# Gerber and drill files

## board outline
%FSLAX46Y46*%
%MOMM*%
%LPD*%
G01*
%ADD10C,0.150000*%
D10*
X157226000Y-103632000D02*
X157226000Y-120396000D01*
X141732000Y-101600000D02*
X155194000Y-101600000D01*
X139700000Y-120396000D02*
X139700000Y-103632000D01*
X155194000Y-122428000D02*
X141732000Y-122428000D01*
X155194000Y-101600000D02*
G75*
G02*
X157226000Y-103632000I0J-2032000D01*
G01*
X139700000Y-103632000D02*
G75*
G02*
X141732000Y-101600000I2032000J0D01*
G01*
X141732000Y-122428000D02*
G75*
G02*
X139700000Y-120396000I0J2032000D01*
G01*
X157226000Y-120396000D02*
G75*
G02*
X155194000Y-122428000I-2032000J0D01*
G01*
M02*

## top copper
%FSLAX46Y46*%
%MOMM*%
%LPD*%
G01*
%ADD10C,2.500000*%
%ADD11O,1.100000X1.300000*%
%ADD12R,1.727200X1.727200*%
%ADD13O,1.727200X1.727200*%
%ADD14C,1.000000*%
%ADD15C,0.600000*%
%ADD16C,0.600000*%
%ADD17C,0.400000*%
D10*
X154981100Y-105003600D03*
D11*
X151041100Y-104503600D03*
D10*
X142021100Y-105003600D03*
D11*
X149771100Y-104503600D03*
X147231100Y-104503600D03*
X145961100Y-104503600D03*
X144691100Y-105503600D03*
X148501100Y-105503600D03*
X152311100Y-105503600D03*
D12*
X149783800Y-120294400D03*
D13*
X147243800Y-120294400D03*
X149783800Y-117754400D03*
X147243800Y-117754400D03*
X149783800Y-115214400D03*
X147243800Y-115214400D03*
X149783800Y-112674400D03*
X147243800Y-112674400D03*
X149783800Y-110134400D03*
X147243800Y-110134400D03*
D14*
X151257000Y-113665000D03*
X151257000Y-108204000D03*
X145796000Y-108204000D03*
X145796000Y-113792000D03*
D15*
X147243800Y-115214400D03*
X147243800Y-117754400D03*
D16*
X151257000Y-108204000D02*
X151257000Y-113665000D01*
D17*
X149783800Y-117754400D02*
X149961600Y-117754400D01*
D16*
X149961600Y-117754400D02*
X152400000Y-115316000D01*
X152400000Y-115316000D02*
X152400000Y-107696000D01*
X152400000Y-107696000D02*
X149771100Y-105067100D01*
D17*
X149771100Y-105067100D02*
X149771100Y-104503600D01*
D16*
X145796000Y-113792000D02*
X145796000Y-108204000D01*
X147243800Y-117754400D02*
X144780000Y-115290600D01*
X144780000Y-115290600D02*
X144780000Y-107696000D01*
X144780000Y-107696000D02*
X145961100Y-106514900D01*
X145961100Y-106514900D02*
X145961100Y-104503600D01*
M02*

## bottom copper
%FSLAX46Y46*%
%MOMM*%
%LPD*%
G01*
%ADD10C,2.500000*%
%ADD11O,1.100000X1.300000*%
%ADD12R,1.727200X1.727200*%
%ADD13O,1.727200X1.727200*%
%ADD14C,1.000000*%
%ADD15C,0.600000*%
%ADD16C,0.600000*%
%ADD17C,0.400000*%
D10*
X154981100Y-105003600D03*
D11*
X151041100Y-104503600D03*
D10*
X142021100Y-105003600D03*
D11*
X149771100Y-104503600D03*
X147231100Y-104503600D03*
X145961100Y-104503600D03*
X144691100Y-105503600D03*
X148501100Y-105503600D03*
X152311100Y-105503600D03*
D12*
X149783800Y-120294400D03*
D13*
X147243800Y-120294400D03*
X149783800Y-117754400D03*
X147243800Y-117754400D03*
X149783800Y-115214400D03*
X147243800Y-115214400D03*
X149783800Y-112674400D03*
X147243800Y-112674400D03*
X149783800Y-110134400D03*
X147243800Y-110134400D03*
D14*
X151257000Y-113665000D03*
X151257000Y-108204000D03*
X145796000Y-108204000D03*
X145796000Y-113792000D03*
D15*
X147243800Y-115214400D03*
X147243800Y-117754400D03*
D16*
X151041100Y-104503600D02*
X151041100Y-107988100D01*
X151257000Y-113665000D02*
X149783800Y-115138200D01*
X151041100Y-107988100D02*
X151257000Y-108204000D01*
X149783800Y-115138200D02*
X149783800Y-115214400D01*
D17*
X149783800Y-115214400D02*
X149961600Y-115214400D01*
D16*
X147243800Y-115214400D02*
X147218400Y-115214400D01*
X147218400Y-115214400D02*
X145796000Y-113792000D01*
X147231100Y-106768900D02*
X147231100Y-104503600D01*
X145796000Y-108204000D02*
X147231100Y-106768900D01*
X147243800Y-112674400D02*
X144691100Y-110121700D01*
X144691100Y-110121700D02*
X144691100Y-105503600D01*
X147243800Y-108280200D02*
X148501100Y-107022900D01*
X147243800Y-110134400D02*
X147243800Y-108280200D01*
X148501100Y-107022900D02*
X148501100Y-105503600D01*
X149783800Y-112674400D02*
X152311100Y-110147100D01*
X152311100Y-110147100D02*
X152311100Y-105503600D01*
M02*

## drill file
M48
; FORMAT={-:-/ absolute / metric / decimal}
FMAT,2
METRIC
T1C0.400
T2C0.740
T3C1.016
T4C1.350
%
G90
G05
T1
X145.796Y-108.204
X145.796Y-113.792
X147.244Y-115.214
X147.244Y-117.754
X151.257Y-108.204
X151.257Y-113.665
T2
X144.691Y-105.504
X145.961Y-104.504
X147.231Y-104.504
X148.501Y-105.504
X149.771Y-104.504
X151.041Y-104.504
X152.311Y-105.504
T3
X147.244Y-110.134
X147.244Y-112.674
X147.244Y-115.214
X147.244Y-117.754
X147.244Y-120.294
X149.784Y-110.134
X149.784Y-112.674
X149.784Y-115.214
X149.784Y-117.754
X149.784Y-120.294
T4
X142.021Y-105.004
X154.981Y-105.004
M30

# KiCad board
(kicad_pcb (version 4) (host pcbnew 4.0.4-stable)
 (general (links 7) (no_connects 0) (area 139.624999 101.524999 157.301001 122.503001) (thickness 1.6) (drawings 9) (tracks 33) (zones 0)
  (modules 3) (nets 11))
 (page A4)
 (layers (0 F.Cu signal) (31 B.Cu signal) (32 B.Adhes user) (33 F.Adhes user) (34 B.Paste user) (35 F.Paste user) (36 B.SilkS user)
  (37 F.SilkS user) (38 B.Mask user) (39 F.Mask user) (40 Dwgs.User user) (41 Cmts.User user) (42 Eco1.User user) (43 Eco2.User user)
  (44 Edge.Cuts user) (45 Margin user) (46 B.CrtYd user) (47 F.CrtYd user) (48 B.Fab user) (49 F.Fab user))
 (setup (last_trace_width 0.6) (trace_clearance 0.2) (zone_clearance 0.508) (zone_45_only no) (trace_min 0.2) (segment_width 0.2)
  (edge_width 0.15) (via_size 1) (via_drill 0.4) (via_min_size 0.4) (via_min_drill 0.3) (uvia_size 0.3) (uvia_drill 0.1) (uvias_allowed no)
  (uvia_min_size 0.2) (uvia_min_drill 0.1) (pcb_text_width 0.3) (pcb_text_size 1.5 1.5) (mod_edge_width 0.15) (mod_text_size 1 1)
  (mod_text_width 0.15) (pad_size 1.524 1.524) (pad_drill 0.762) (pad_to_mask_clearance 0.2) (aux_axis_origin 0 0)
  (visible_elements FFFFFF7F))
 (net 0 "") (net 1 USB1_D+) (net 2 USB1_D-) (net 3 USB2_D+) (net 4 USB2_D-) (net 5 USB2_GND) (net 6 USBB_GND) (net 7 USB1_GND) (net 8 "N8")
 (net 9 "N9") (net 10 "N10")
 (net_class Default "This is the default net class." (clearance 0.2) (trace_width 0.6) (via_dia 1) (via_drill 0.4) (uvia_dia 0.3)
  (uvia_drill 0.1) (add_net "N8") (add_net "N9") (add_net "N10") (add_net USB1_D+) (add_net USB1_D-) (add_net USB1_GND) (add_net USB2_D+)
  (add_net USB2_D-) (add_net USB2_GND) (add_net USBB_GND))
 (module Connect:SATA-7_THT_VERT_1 (layer F.Cu) (at 148.5011 105.0036)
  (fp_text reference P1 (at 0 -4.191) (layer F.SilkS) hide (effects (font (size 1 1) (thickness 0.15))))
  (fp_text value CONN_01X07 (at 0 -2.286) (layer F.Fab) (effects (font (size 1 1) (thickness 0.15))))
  (pad 9 thru_hole circle (at 6.48 0) (size 2.5 2.5) (drill 1.35) (layers *.Cu *.Mask F.SilkS))
  (pad 2 thru_hole oval (at 2.54 -0.5) (size 1.1 1.3) (drill 0.74) (layers *.Cu *.Mask F.SilkS) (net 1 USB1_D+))
  (pad 8 thru_hole circle (at -6.48 0) (size 2.5 2.5) (drill 1.35) (layers *.Cu *.Mask F.SilkS))
  (pad 3 thru_hole oval (at 1.27 -0.5) (size 1.1 1.3) (drill 0.74) (layers *.Cu *.Mask F.SilkS) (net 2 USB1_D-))
  (pad 5 thru_hole oval (at -1.27 -0.5) (size 1.1 1.3) (drill 0.74) (layers *.Cu *.Mask F.SilkS) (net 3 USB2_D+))
  (pad 6 thru_hole oval (at -2.54 -0.5) (size 1.1 1.3) (drill 0.74) (layers *.Cu *.Mask F.SilkS) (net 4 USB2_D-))
  (pad 7 thru_hole oval (at -3.81 0.5) (size 1.1 1.3) (drill 0.74) (layers *.Cu *.Mask F.SilkS) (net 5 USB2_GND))
  (pad 4 thru_hole oval (at 0 0.5) (size 1.1 1.3) (drill 0.74) (layers *.Cu *.Mask F.SilkS) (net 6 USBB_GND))
  (pad 1 thru_hole oval (at 3.81 0.5) (size 1.1 1.3) (drill 0.74) (layers *.Cu *.Mask F.SilkS) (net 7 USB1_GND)))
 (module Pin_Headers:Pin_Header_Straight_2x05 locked (layer F.Cu) (at 149.7838 120.2944 180)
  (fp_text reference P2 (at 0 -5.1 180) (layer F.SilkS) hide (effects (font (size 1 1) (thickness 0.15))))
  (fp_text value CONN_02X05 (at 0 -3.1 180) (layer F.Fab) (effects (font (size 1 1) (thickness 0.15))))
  (pad 1 thru_hole rect (at 0 0 180) (size 1.7272 1.7272) (drill 1.016) (layers *.Cu *.Mask F.SilkS) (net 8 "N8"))
  (pad 2 thru_hole oval (at 2.54 0 180) (size 1.7272 1.7272) (drill 1.016) (layers *.Cu *.Mask F.SilkS) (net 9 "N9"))
  (pad 3 thru_hole oval (at 0 2.54 180) (size 1.7272 1.7272) (drill 1.016) (layers *.Cu *.Mask F.SilkS) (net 2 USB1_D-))
  (pad 4 thru_hole oval (at 2.54 2.54 180) (size 1.7272 1.7272) (drill 1.016) (layers *.Cu *.Mask F.SilkS) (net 4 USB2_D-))
  (pad 5 thru_hole oval (at 0 5.08 180) (size 1.7272 1.7272) (drill 1.016) (layers *.Cu *.Mask F.SilkS) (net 1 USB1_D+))
  (pad 6 thru_hole oval (at 2.54 5.08 180) (size 1.7272 1.7272) (drill 1.016) (layers *.Cu *.Mask F.SilkS) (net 3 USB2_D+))
  (pad 7 thru_hole oval (at 0 7.62 180) (size 1.7272 1.7272) (drill 1.016) (layers *.Cu *.Mask F.SilkS) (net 7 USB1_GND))
  (pad 8 thru_hole oval (at 2.54 7.62 180) (size 1.7272 1.7272) (drill 1.016) (layers *.Cu *.Mask F.SilkS) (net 5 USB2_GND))
  (pad 9 thru_hole oval (at 0 10.16 180) (size 1.7272 1.7272) (drill 1.016) (layers *.Cu *.Mask F.SilkS) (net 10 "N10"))
  (pad 10 thru_hole oval (at 2.54 10.16 180) (size 1.7272 1.7272) (drill 1.016) (layers *.Cu *.Mask F.SilkS) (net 6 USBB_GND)))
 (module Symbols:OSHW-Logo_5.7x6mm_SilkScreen (layer F.Cu) (at 142.875 117.221)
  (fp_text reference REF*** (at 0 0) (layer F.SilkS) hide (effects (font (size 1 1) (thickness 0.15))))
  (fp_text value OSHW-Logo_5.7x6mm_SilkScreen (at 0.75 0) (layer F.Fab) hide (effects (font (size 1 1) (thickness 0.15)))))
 (gr_line (start 157.226 103.632) (end 157.226 120.396) (angle 90) (layer Edge.Cuts) (width 0.15))
 (gr_line (start 141.732 101.6) (end 155.194 101.6) (angle 90) (layer Edge.Cuts) (width 0.15))
 (gr_line (start 139.7 120.396) (end 139.7 103.632) (angle 90) (layer Edge.Cuts) (width 0.15))
 (gr_line (start 155.194 122.428) (end 141.732 122.428) (angle 90) (layer Edge.Cuts) (width 0.15))
 (gr_arc (start 155.194 103.632) (end 155.194 101.6) (angle 90) (layer Edge.Cuts) (width 0.15))
 (gr_arc (start 141.732 103.632) (end 139.7 103.632) (angle 90) (layer Edge.Cuts) (width 0.15))
 (gr_arc (start 141.732 120.396) (end 141.732 122.428) (angle 90) (layer Edge.Cuts) (width 0.15))
 (gr_arc (start 155.194 120.396) (end 157.226 120.396) (angle 90) (layer Edge.Cuts) (width 0.15))
 (segment (start 151.0411 104.5036) (end 151.0411 107.9881) (width 0.6) (layer B.Cu) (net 1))
 (segment (start 151.257 113.665) (end 149.7838 115.1382) (width 0.6) (layer B.Cu) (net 1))
 (segment (start 151.257 108.204) (end 151.257 113.665) (width 0.6) (layer F.Cu) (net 1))
 (segment (start 151.0411 107.9881) (end 151.257 108.204) (width 0.6) (layer B.Cu) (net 1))
 (segment (start 149.7838 115.1382) (end 149.7838 115.2144) (width 0.6) (layer B.Cu) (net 1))
 (segment (start 149.7838 115.2144) (end 149.9616 115.2144) (width 0.4) (layer B.Cu) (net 1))
 (segment (start 149.7838 117.7544) (end 149.9616 117.7544) (width 0.4) (layer F.Cu) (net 2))
 (segment (start 149.9616 117.7544) (end 152.4 115.316) (width 0.6) (layer F.Cu) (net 2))
 (segment (start 152.4 115.316) (end 152.4 107.696) (width 0.6) (layer F.Cu) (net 2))
 (segment (start 152.4 107.696) (end 149.7711 105.0671) (width 0.6) (layer F.Cu) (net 2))
 (segment (start 149.7711 105.0671) (end 149.7711 104.5036) (width 0.4) (layer F.Cu) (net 2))
 (segment (start 147.2438 115.2144) (end 147.2184 115.2144) (width 0.6) (layer B.Cu) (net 3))
 (segment (start 147.2184 115.2144) (end 145.796 113.792) (width 0.6) (layer B.Cu) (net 3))
 (segment (start 147.2311 106.7689) (end 147.2311 104.5036) (width 0.6) (layer B.Cu) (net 3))
 (segment (start 145.796 108.204) (end 147.2311 106.7689) (width 0.6) (layer B.Cu) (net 3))
 (segment (start 145.796 113.792) (end 145.796 108.204) (width 0.6) (layer F.Cu) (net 3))
 (segment (start 147.2438 117.7544) (end 144.78 115.2906) (width 0.6) (layer F.Cu) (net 4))
 (segment (start 144.78 115.2906) (end 144.78 107.696) (width 0.6) (layer F.Cu) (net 4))
 (segment (start 144.78 107.696) (end 145.9611 106.5149) (width 0.6) (layer F.Cu) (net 4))
 (segment (start 145.9611 106.5149) (end 145.9611 104.5036) (width 0.6) (layer F.Cu) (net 4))
 (segment (start 147.2438 112.6744) (end 144.6911 110.1217) (width 0.6) (layer B.Cu) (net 5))
 (segment (start 144.6911 110.1217) (end 144.6911 105.5036) (width 0.6) (layer B.Cu) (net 5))
 (segment (start 147.2438 108.2802) (end 148.5011 107.0229) (width 0.6) (layer B.Cu) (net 6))
 (segment (start 147.2438 110.1344) (end 147.2438 108.2802) (width 0.6) (layer B.Cu) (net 6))
 (segment (start 148.5011 107.0229) (end 148.5011 105.5036) (width 0.6) (layer B.Cu) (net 6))
 (segment (start 149.7838 112.6744) (end 152.3111 110.1471) (width 0.6) (layer B.Cu) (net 7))
 (segment (start 152.3111 110.1471) (end 152.3111 105.5036) (width 0.6) (layer B.Cu) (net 7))
 (via (at 151.257 113.665) (size 1) (drill 0.4) (layers F.Cu B.Cu) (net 1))
 (via (at 151.257 108.204) (size 1) (drill 0.4) (layers F.Cu B.Cu) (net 1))
 (via (at 145.796 108.204) (size 1) (drill 0.4) (layers F.Cu B.Cu) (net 3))
 (via (at 145.796 113.792) (size 1) (drill 0.4) (layers F.Cu B.Cu) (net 3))
 (via (at 147.2438 115.2144) (size 0.6) (drill 0.4) (layers F.Cu B.Cu) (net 3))
 (via (at 147.2438 117.7544) (size 0.6) (drill 0.4) (layers F.Cu B.Cu) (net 4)))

